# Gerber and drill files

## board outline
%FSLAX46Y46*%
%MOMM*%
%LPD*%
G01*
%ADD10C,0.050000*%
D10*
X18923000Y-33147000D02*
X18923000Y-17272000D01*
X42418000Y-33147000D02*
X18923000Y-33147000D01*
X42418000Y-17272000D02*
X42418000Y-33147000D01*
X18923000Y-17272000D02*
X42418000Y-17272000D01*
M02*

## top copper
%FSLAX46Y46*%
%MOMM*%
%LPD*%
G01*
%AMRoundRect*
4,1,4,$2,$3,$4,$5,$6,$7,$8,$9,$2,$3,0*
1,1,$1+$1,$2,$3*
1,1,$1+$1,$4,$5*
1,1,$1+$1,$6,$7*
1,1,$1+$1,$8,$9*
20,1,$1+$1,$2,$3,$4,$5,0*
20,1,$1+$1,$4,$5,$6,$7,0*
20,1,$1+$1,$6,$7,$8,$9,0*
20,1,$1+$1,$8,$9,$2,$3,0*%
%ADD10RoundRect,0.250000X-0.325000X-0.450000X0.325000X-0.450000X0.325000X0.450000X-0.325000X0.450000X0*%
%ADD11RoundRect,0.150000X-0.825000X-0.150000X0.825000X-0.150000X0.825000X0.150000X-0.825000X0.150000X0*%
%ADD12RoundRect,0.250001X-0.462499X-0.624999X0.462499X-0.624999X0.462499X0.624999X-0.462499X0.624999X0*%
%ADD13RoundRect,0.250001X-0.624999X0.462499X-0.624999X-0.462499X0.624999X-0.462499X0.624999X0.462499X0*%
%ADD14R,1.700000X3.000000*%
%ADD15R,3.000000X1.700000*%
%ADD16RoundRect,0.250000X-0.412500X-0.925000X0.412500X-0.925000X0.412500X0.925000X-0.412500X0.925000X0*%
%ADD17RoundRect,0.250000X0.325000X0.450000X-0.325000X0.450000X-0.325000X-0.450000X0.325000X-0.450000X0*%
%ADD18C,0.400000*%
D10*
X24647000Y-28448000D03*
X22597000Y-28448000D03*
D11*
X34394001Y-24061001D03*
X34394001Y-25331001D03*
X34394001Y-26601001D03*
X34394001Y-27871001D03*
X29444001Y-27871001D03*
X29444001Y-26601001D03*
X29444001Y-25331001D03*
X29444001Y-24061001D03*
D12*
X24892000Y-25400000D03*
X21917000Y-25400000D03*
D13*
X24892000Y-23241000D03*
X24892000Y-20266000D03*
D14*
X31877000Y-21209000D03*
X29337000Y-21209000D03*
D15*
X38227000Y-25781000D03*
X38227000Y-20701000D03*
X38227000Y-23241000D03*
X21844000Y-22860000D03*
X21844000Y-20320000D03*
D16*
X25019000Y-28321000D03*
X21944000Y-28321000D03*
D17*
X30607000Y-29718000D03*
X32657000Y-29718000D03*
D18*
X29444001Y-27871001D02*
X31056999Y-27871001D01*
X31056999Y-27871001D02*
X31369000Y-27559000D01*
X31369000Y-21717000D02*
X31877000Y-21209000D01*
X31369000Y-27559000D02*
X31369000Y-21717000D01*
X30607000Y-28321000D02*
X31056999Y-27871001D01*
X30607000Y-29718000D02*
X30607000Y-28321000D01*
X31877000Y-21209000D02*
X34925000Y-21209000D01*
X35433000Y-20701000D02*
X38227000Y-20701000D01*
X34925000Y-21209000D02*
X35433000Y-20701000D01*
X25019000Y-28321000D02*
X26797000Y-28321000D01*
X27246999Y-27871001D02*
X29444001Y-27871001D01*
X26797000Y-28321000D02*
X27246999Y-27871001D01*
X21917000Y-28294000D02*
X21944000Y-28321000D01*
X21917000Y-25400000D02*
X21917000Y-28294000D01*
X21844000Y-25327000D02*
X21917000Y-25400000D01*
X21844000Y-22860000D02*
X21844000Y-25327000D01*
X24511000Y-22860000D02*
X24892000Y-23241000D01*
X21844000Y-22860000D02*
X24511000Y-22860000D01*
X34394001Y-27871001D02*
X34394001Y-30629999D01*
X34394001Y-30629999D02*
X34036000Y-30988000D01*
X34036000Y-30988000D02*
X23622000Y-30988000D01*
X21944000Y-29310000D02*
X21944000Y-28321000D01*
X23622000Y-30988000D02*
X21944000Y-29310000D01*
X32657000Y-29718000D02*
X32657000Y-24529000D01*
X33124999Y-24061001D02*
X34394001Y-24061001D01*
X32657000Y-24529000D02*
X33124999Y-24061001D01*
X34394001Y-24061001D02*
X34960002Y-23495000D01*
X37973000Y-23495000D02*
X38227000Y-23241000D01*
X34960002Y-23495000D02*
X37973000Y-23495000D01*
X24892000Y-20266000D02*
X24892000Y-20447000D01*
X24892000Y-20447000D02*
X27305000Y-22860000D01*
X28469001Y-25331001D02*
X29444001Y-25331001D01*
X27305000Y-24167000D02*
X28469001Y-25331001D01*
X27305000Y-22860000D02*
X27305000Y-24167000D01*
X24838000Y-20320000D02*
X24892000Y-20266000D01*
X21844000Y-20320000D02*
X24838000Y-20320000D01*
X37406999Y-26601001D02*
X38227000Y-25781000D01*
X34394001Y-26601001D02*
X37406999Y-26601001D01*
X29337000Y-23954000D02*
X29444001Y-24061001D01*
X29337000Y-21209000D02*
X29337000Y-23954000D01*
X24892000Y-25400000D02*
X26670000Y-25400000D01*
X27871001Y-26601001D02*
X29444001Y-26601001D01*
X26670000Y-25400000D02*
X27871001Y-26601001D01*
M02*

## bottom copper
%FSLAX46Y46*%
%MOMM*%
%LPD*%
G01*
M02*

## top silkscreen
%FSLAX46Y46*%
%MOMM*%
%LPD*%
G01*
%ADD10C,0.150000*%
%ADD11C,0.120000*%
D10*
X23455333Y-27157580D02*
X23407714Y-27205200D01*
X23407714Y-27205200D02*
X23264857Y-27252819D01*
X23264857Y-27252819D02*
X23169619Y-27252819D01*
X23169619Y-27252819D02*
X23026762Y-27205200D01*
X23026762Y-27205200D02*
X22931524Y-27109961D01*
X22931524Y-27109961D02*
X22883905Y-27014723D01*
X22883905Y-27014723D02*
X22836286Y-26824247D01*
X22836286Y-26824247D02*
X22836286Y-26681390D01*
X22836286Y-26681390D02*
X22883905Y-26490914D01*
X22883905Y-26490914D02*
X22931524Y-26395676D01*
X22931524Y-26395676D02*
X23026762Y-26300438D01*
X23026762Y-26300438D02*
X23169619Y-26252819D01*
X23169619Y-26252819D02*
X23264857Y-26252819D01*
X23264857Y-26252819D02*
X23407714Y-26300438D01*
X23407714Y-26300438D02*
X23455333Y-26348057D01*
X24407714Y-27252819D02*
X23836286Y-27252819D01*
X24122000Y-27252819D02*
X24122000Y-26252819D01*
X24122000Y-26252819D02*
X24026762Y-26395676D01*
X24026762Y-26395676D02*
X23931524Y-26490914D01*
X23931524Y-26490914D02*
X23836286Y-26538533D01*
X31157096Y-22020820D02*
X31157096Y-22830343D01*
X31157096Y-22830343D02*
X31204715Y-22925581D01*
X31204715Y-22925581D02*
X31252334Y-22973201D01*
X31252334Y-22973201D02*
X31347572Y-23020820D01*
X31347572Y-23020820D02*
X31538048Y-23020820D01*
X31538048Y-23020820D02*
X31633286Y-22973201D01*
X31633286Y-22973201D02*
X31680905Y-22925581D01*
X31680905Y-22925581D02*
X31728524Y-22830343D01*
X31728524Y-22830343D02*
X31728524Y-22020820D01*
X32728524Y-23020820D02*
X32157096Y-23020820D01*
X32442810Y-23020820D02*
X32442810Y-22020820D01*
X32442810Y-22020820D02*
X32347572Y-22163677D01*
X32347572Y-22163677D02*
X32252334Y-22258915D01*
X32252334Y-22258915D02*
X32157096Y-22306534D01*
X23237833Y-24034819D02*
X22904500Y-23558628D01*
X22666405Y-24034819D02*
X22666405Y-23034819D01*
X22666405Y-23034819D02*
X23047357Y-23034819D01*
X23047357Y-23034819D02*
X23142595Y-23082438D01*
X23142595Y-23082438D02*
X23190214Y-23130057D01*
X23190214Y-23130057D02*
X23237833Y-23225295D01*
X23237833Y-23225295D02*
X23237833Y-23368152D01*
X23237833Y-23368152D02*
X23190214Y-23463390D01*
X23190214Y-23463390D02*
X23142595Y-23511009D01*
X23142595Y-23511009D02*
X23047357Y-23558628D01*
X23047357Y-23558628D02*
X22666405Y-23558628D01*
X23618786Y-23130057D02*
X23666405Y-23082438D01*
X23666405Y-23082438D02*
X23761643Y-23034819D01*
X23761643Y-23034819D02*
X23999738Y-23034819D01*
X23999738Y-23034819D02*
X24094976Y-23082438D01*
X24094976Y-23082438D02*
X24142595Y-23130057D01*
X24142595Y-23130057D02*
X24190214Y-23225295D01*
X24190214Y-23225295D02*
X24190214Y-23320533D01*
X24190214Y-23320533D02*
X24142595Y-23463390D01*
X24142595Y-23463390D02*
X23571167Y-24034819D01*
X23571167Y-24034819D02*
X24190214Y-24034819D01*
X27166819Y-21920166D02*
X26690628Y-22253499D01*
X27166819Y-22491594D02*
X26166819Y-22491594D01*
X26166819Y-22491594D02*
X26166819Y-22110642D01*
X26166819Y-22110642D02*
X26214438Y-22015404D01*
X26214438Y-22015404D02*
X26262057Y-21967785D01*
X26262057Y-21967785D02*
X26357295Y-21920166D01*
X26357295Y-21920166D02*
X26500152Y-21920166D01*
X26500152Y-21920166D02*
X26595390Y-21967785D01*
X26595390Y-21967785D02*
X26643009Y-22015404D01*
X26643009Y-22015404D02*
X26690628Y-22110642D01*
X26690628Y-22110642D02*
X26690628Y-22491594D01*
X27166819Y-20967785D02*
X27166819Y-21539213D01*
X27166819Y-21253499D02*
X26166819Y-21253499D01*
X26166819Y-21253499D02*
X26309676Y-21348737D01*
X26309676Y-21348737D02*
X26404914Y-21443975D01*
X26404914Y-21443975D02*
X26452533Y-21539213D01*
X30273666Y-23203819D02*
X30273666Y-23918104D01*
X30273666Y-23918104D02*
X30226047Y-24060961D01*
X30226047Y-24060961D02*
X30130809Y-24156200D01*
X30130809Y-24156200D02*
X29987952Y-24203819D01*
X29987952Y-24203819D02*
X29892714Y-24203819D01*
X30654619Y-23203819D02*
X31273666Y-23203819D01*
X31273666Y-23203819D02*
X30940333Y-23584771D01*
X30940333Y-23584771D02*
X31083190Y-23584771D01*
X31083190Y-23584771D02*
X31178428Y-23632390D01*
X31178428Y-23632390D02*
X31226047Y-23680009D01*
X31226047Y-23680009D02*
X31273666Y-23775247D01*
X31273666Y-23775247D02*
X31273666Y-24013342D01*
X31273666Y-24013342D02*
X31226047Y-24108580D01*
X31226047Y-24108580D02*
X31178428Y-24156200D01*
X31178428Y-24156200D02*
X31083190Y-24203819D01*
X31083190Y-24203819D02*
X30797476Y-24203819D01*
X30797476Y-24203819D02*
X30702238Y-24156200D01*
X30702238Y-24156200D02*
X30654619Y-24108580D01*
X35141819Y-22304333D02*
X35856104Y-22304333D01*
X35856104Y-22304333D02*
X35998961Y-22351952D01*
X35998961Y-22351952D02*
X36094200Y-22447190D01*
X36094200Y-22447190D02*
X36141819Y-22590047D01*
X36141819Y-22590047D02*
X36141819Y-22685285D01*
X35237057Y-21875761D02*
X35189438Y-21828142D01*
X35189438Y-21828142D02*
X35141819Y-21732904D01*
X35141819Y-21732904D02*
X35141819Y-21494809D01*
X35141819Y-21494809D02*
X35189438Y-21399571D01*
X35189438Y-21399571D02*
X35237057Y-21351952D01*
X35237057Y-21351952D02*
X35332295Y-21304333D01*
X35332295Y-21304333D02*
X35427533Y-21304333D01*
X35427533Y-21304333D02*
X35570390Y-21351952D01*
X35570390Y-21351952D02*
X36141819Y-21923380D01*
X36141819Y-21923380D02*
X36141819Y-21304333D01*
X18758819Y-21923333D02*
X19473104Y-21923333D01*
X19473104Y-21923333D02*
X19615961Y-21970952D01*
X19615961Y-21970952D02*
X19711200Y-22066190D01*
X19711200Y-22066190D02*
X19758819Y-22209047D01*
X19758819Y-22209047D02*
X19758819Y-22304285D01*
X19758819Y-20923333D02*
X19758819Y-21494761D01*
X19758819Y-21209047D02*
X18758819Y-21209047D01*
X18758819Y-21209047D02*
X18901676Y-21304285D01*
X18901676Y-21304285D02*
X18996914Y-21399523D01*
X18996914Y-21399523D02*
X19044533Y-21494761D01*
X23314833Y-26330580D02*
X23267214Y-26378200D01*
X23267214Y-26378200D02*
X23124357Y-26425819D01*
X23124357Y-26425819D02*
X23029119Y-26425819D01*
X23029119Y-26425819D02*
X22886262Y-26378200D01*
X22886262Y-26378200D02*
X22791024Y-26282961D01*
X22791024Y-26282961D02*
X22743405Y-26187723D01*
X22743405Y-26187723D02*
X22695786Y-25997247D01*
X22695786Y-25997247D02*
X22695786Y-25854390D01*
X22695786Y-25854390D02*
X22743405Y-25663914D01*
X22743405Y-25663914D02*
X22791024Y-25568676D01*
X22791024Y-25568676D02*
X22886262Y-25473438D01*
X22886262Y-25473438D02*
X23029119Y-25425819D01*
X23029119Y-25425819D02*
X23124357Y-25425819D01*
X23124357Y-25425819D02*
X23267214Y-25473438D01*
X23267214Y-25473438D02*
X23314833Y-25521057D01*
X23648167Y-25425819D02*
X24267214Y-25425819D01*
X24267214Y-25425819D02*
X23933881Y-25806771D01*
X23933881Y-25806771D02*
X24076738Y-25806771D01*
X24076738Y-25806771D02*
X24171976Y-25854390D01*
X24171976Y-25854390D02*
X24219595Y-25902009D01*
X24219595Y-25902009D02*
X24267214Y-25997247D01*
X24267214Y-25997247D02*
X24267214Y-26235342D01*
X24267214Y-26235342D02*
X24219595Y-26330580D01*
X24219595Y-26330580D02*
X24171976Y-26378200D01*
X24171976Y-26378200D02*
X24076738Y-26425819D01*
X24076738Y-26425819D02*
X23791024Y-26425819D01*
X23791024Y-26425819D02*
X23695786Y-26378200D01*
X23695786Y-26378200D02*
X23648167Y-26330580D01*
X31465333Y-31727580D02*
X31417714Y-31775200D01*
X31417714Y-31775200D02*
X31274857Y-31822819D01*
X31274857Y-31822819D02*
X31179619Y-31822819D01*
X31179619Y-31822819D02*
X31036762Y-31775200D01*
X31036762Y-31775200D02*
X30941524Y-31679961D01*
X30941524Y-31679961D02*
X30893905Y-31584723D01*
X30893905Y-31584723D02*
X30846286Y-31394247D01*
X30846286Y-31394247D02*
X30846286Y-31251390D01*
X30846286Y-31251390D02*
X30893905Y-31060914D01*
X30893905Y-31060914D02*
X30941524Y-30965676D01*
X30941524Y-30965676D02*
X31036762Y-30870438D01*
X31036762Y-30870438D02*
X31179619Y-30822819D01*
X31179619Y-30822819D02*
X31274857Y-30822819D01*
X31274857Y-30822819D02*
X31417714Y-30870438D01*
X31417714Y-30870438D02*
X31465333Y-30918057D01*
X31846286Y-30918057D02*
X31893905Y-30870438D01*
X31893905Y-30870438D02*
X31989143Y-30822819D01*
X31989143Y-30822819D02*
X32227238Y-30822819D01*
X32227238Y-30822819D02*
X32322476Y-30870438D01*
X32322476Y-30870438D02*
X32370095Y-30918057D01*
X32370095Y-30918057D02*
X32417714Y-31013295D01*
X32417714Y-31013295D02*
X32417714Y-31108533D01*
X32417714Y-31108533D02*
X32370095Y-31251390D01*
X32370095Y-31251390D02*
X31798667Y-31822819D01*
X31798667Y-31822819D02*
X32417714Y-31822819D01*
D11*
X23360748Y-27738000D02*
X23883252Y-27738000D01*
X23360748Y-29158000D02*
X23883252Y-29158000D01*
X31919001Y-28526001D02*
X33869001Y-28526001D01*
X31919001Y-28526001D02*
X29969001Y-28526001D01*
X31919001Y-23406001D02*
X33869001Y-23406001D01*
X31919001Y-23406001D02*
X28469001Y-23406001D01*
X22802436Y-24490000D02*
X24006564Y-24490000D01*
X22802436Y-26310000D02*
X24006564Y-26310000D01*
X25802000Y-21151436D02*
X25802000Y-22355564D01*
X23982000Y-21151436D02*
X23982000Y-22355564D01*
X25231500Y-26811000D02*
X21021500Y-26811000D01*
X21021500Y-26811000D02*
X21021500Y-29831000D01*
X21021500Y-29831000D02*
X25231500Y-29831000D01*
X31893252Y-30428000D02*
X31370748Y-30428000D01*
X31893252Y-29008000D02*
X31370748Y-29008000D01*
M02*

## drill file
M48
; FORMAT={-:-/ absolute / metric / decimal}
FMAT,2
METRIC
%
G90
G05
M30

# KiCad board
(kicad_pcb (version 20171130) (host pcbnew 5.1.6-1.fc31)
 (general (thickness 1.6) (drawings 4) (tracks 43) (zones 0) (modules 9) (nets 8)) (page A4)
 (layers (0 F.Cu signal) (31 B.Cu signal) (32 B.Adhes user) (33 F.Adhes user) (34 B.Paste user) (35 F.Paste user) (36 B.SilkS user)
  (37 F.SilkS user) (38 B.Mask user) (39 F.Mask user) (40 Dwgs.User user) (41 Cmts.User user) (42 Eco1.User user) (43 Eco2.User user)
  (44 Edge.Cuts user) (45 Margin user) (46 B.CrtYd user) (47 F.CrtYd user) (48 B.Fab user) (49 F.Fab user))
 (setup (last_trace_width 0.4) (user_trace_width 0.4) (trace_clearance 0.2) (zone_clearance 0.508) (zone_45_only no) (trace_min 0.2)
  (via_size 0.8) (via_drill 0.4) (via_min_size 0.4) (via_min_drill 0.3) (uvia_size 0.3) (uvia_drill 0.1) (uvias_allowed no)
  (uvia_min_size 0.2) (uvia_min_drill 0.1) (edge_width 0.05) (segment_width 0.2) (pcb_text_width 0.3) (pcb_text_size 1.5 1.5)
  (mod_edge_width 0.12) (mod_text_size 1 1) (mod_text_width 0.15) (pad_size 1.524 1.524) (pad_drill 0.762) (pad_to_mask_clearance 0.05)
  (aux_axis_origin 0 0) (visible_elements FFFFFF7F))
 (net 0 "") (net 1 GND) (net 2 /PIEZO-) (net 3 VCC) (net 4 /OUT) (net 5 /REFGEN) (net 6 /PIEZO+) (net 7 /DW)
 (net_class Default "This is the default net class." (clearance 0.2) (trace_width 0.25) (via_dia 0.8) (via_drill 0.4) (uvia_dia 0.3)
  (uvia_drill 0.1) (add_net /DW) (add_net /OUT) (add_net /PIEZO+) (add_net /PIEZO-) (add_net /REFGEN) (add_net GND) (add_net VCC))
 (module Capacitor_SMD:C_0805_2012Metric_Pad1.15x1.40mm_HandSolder (layer F.Cu) (at 23.622 28.448)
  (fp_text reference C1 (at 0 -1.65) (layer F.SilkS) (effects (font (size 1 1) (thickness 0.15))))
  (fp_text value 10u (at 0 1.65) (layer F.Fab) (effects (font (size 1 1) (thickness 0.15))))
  (fp_line (start -0.261252 -0.71) (end 0.261252 -0.71) (layer F.SilkS) (width 0.12))
  (fp_line (start -0.261252 0.71) (end 0.261252 0.71) (layer F.SilkS) (width 0.12))
  (pad 2 smd roundrect (at 1.025 0) (size 1.15 1.4) (layers F.Cu F.Paste F.Mask) (roundrect_rratio 0.217391) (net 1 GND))
  (pad 1 smd roundrect (at -1.025 0) (size 1.15 1.4) (layers F.Cu F.Paste F.Mask) (roundrect_rratio 0.217391) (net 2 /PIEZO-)))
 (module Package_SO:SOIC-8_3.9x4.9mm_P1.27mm (layer F.Cu) (at 31.919001 25.966001)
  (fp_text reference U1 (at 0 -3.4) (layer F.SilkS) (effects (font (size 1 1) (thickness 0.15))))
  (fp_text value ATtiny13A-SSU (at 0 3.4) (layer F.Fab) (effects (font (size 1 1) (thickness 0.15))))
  (fp_line (start 0 2.56) (end 1.95 2.56) (layer F.SilkS) (width 0.12))
  (fp_line (start 0 2.56) (end -1.95 2.56) (layer F.SilkS) (width 0.12))
  (fp_line (start 0 -2.56) (end 1.95 -2.56) (layer F.SilkS) (width 0.12))
  (fp_line (start 0 -2.56) (end -3.45 -2.56) (layer F.SilkS) (width 0.12))
  (pad 8 smd roundrect (at 2.475 -1.905) (size 1.95 0.6) (layers F.Cu F.Paste F.Mask) (roundrect_rratio 0.25) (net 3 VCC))
  (pad 7 smd roundrect (at 2.475 -0.635) (size 1.95 0.6) (layers F.Cu F.Paste F.Mask) (roundrect_rratio 0.25))
  (pad 6 smd roundrect (at 2.475 0.635) (size 1.95 0.6) (layers F.Cu F.Paste F.Mask) (roundrect_rratio 0.25) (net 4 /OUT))
  (pad 5 smd roundrect (at 2.475 1.905) (size 1.95 0.6) (layers F.Cu F.Paste F.Mask) (roundrect_rratio 0.25) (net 2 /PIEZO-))
  (pad 4 smd roundrect (at -2.475 1.905) (size 1.95 0.6) (layers F.Cu F.Paste F.Mask) (roundrect_rratio 0.25) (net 1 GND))
  (pad 3 smd roundrect (at -2.475 0.635) (size 1.95 0.6) (layers F.Cu F.Paste F.Mask) (roundrect_rratio 0.25) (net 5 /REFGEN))
  (pad 2 smd roundrect (at -2.475 -0.635) (size 1.95 0.6) (layers F.Cu F.Paste F.Mask) (roundrect_rratio 0.25) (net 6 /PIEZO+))
  (pad 1 smd roundrect (at -2.475 -1.905) (size 1.95 0.6) (layers F.Cu F.Paste F.Mask) (roundrect_rratio 0.25) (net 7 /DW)))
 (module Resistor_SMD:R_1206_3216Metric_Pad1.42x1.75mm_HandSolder (layer F.Cu) (at 23.4045 25.4)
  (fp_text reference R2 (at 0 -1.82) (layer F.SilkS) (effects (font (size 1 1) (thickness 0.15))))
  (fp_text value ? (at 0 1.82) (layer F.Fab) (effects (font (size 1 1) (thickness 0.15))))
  (fp_line (start -0.602064 -0.91) (end 0.602064 -0.91) (layer F.SilkS) (width 0.12))
  (fp_line (start -0.602064 0.91) (end 0.602064 0.91) (layer F.SilkS) (width 0.12))
  (pad 2 smd roundrect (at 1.4875 0) (size 1.425 1.75) (layers F.Cu F.Paste F.Mask) (roundrect_rratio 0.175439) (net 5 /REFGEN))
  (pad 1 smd roundrect (at -1.4875 0) (size 1.425 1.75) (layers F.Cu F.Paste F.Mask) (roundrect_rratio 0.175439) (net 2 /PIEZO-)))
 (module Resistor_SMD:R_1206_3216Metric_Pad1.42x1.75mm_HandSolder (layer F.Cu) (at 24.892 21.7535 270)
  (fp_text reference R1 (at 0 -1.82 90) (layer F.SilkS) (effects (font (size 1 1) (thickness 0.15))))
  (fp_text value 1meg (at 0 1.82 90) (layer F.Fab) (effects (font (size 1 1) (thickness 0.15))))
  (fp_line (start -0.602064 -0.91) (end 0.602064 -0.91) (layer F.SilkS) (width 0.12))
  (fp_line (start -0.602064 0.91) (end 0.602064 0.91) (layer F.SilkS) (width 0.12))
  (pad 2 smd roundrect (at 1.4875 0 270) (size 1.425 1.75) (layers F.Cu F.Paste F.Mask) (roundrect_rratio 0.175439) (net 2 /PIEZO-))
  (pad 1 smd roundrect (at -1.4875 0 270) (size 1.425 1.75) (layers F.Cu F.Paste F.Mask) (roundrect_rratio 0.175439) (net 6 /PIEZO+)))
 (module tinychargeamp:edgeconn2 (layer F.Cu) (at 30.607 21.209 90)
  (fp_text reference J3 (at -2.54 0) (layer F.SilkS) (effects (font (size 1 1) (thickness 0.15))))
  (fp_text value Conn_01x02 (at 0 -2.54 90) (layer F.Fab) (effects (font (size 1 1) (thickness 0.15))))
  (pad 2 smd rect (at 0 1.27 90) (size 3 1.7) (layers F.Cu F.Paste F.Mask) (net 1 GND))
  (pad 1 smd rect (at 0 -1.27 90) (size 3 1.7) (layers F.Cu F.Paste F.Mask) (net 7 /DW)))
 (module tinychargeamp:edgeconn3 (layer F.Cu) (at 38.227 21.971)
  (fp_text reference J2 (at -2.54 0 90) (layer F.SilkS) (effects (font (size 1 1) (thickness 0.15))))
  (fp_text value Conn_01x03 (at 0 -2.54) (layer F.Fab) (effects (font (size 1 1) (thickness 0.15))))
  (pad 3 smd rect (at 0 3.81) (size 3 1.7) (layers F.Cu F.Paste F.Mask) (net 4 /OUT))
  (pad 1 smd rect (at 0 -1.27) (size 3 1.7) (layers F.Cu F.Paste F.Mask) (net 1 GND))
  (pad 2 smd rect (at 0 1.27) (size 3 1.7) (layers F.Cu F.Paste F.Mask) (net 3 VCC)))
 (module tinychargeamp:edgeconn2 (layer F.Cu) (at 21.844 21.59)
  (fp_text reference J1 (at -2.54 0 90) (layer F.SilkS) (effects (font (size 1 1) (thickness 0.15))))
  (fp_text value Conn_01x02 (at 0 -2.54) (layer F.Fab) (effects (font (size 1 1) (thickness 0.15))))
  (pad 2 smd rect (at 0 1.27) (size 3 1.7) (layers F.Cu F.Paste F.Mask) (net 2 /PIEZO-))
  (pad 1 smd rect (at 0 -1.27) (size 3 1.7) (layers F.Cu F.Paste F.Mask) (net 6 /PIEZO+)))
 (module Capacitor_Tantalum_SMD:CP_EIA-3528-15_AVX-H (layer F.Cu) (at 23.4815 28.321)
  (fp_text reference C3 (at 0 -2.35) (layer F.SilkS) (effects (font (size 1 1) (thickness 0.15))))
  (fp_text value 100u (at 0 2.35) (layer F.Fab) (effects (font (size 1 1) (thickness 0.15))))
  (fp_line (start 1.75 -1.51) (end -2.46 -1.51) (layer F.SilkS) (width 0.12))
  (fp_line (start -2.46 -1.51) (end -2.46 1.51) (layer F.SilkS) (width 0.12))
  (fp_line (start -2.46 1.51) (end 1.75 1.51) (layer F.SilkS) (width 0.12))
  (pad 2 smd roundrect (at 1.5375 0) (size 1.325 2.35) (layers F.Cu F.Paste F.Mask) (roundrect_rratio 0.188679) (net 1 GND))
  (pad 1 smd roundrect (at -1.5375 0) (size 1.325 2.35) (layers F.Cu F.Paste F.Mask) (roundrect_rratio 0.188679) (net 2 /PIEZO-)))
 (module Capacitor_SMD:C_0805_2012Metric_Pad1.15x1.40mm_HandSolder (layer F.Cu) (at 31.632 29.718 180)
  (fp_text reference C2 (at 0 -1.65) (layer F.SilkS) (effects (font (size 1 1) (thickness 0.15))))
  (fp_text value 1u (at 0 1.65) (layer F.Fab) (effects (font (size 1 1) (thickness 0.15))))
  (fp_line (start -0.261252 -0.71) (end 0.261252 -0.71) (layer F.SilkS) (width 0.12))
  (fp_line (start -0.261252 0.71) (end 0.261252 0.71) (layer F.SilkS) (width 0.12))
  (pad 2 smd roundrect (at 1.025 0 180) (size 1.15 1.4) (layers F.Cu F.Paste F.Mask) (roundrect_rratio 0.217391) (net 1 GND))
  (pad 1 smd roundrect (at -1.025 0 180) (size 1.15 1.4) (layers F.Cu F.Paste F.Mask) (roundrect_rratio 0.217391) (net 3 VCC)))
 (gr_line (start 18.923 33.147) (end 18.923 17.272) (layer Edge.Cuts) (width 0.05))
 (gr_line (start 42.418 33.147) (end 18.923 33.147) (layer Edge.Cuts) (width 0.05))
 (gr_line (start 42.418 17.272) (end 42.418 33.147) (layer Edge.Cuts) (width 0.05))
 (gr_line (start 18.923 17.272) (end 42.418 17.272) (layer Edge.Cuts) (width 0.05))
 (segment (start 29.444001 27.871001) (end 31.056999 27.871001) (width 0.4) (layer F.Cu) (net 1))
 (segment (start 31.056999 27.871001) (end 31.369 27.559) (width 0.4) (layer F.Cu) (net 1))
 (segment (start 31.369 21.717) (end 31.877 21.209) (width 0.4) (layer F.Cu) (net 1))
 (segment (start 31.369 27.559) (end 31.369 21.717) (width 0.4) (layer F.Cu) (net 1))
 (segment (start 30.607 28.321) (end 31.056999 27.871001) (width 0.4) (layer F.Cu) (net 1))
 (segment (start 30.607 29.718) (end 30.607 28.321) (width 0.4) (layer F.Cu) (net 1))
 (segment (start 31.877 21.209) (end 34.925 21.209) (width 0.4) (layer F.Cu) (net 1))
 (segment (start 35.433 20.701) (end 38.227 20.701) (width 0.4) (layer F.Cu) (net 1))
 (segment (start 34.925 21.209) (end 35.433 20.701) (width 0.4) (layer F.Cu) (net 1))
 (segment (start 25.019 28.321) (end 26.797 28.321) (width 0.4) (layer F.Cu) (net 1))
 (segment (start 27.246999 27.871001) (end 29.444001 27.871001) (width 0.4) (layer F.Cu) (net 1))
 (segment (start 26.797 28.321) (end 27.246999 27.871001) (width 0.4) (layer F.Cu) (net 1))
 (segment (start 21.917 28.294) (end 21.944 28.321) (width 0.4) (layer F.Cu) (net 2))
 (segment (start 21.917 25.4) (end 21.917 28.294) (width 0.4) (layer F.Cu) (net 2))
 (segment (start 21.844 25.327) (end 21.917 25.4) (width 0.4) (layer F.Cu) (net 2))
 (segment (start 21.844 22.86) (end 21.844 25.327) (width 0.4) (layer F.Cu) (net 2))
 (segment (start 24.511 22.86) (end 24.892 23.241) (width 0.4) (layer F.Cu) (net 2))
 (segment (start 21.844 22.86) (end 24.511 22.86) (width 0.4) (layer F.Cu) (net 2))
 (segment (start 34.394001 27.871001) (end 34.394001 30.629999) (width 0.4) (layer F.Cu) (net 2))
 (segment (start 34.394001 30.629999) (end 34.036 30.988) (width 0.4) (layer F.Cu) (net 2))
 (segment (start 34.036 30.988) (end 23.622 30.988) (width 0.4) (layer F.Cu) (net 2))
 (segment (start 21.944 29.31) (end 21.944 28.321) (width 0.4) (layer F.Cu) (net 2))
 (segment (start 23.622 30.988) (end 21.944 29.31) (width 0.4) (layer F.Cu) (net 2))
 (segment (start 32.657 29.718) (end 32.657 24.529) (width 0.4) (layer F.Cu) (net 3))
 (segment (start 33.124999 24.061001) (end 34.394001 24.061001) (width 0.4) (layer F.Cu) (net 3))
 (segment (start 32.657 24.529) (end 33.124999 24.061001) (width 0.4) (layer F.Cu) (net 3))
 (segment (start 34.394001 24.061001) (end 34.960002 23.495) (width 0.4) (layer F.Cu) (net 3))
 (segment (start 37.973 23.495) (end 38.227 23.241) (width 0.4) (layer F.Cu) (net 3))
 (segment (start 34.960002 23.495) (end 37.973 23.495) (width 0.4) (layer F.Cu) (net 3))
 (segment (start 24.892 20.266) (end 24.892 20.447) (width 0.4) (layer F.Cu) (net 6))
 (segment (start 24.892 20.447) (end 27.305 22.86) (width 0.4) (layer F.Cu) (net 6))
 (segment (start 28.469001 25.331001) (end 29.444001 25.331001) (width 0.4) (layer F.Cu) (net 6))
 (segment (start 27.305 24.167) (end 28.469001 25.331001) (width 0.4) (layer F.Cu) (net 6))
 (segment (start 27.305 22.86) (end 27.305 24.167) (width 0.4) (layer F.Cu) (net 6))
 (segment (start 24.838 20.32) (end 24.892 20.266) (width 0.4) (layer F.Cu) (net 6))
 (segment (start 21.844 20.32) (end 24.838 20.32) (width 0.4) (layer F.Cu) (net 6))
 (segment (start 37.406999 26.601001) (end 38.227 25.781) (width 0.4) (layer F.Cu) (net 4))
 (segment (start 34.394001 26.601001) (end 37.406999 26.601001) (width 0.4) (layer F.Cu) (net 4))
 (segment (start 29.337 23.954) (end 29.444001 24.061001) (width 0.4) (layer F.Cu) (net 7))
 (segment (start 29.337 21.209) (end 29.337 23.954) (width 0.4) (layer F.Cu) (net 7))
 (segment (start 24.892 25.4) (end 26.67 25.4) (width 0.4) (layer F.Cu) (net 5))
 (segment (start 27.871001 26.601001) (end 29.444001 26.601001) (width 0.4) (layer F.Cu) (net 5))
 (segment (start 26.67 25.4) (end 27.871001 26.601001) (width 0.4) (layer F.Cu) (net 5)))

